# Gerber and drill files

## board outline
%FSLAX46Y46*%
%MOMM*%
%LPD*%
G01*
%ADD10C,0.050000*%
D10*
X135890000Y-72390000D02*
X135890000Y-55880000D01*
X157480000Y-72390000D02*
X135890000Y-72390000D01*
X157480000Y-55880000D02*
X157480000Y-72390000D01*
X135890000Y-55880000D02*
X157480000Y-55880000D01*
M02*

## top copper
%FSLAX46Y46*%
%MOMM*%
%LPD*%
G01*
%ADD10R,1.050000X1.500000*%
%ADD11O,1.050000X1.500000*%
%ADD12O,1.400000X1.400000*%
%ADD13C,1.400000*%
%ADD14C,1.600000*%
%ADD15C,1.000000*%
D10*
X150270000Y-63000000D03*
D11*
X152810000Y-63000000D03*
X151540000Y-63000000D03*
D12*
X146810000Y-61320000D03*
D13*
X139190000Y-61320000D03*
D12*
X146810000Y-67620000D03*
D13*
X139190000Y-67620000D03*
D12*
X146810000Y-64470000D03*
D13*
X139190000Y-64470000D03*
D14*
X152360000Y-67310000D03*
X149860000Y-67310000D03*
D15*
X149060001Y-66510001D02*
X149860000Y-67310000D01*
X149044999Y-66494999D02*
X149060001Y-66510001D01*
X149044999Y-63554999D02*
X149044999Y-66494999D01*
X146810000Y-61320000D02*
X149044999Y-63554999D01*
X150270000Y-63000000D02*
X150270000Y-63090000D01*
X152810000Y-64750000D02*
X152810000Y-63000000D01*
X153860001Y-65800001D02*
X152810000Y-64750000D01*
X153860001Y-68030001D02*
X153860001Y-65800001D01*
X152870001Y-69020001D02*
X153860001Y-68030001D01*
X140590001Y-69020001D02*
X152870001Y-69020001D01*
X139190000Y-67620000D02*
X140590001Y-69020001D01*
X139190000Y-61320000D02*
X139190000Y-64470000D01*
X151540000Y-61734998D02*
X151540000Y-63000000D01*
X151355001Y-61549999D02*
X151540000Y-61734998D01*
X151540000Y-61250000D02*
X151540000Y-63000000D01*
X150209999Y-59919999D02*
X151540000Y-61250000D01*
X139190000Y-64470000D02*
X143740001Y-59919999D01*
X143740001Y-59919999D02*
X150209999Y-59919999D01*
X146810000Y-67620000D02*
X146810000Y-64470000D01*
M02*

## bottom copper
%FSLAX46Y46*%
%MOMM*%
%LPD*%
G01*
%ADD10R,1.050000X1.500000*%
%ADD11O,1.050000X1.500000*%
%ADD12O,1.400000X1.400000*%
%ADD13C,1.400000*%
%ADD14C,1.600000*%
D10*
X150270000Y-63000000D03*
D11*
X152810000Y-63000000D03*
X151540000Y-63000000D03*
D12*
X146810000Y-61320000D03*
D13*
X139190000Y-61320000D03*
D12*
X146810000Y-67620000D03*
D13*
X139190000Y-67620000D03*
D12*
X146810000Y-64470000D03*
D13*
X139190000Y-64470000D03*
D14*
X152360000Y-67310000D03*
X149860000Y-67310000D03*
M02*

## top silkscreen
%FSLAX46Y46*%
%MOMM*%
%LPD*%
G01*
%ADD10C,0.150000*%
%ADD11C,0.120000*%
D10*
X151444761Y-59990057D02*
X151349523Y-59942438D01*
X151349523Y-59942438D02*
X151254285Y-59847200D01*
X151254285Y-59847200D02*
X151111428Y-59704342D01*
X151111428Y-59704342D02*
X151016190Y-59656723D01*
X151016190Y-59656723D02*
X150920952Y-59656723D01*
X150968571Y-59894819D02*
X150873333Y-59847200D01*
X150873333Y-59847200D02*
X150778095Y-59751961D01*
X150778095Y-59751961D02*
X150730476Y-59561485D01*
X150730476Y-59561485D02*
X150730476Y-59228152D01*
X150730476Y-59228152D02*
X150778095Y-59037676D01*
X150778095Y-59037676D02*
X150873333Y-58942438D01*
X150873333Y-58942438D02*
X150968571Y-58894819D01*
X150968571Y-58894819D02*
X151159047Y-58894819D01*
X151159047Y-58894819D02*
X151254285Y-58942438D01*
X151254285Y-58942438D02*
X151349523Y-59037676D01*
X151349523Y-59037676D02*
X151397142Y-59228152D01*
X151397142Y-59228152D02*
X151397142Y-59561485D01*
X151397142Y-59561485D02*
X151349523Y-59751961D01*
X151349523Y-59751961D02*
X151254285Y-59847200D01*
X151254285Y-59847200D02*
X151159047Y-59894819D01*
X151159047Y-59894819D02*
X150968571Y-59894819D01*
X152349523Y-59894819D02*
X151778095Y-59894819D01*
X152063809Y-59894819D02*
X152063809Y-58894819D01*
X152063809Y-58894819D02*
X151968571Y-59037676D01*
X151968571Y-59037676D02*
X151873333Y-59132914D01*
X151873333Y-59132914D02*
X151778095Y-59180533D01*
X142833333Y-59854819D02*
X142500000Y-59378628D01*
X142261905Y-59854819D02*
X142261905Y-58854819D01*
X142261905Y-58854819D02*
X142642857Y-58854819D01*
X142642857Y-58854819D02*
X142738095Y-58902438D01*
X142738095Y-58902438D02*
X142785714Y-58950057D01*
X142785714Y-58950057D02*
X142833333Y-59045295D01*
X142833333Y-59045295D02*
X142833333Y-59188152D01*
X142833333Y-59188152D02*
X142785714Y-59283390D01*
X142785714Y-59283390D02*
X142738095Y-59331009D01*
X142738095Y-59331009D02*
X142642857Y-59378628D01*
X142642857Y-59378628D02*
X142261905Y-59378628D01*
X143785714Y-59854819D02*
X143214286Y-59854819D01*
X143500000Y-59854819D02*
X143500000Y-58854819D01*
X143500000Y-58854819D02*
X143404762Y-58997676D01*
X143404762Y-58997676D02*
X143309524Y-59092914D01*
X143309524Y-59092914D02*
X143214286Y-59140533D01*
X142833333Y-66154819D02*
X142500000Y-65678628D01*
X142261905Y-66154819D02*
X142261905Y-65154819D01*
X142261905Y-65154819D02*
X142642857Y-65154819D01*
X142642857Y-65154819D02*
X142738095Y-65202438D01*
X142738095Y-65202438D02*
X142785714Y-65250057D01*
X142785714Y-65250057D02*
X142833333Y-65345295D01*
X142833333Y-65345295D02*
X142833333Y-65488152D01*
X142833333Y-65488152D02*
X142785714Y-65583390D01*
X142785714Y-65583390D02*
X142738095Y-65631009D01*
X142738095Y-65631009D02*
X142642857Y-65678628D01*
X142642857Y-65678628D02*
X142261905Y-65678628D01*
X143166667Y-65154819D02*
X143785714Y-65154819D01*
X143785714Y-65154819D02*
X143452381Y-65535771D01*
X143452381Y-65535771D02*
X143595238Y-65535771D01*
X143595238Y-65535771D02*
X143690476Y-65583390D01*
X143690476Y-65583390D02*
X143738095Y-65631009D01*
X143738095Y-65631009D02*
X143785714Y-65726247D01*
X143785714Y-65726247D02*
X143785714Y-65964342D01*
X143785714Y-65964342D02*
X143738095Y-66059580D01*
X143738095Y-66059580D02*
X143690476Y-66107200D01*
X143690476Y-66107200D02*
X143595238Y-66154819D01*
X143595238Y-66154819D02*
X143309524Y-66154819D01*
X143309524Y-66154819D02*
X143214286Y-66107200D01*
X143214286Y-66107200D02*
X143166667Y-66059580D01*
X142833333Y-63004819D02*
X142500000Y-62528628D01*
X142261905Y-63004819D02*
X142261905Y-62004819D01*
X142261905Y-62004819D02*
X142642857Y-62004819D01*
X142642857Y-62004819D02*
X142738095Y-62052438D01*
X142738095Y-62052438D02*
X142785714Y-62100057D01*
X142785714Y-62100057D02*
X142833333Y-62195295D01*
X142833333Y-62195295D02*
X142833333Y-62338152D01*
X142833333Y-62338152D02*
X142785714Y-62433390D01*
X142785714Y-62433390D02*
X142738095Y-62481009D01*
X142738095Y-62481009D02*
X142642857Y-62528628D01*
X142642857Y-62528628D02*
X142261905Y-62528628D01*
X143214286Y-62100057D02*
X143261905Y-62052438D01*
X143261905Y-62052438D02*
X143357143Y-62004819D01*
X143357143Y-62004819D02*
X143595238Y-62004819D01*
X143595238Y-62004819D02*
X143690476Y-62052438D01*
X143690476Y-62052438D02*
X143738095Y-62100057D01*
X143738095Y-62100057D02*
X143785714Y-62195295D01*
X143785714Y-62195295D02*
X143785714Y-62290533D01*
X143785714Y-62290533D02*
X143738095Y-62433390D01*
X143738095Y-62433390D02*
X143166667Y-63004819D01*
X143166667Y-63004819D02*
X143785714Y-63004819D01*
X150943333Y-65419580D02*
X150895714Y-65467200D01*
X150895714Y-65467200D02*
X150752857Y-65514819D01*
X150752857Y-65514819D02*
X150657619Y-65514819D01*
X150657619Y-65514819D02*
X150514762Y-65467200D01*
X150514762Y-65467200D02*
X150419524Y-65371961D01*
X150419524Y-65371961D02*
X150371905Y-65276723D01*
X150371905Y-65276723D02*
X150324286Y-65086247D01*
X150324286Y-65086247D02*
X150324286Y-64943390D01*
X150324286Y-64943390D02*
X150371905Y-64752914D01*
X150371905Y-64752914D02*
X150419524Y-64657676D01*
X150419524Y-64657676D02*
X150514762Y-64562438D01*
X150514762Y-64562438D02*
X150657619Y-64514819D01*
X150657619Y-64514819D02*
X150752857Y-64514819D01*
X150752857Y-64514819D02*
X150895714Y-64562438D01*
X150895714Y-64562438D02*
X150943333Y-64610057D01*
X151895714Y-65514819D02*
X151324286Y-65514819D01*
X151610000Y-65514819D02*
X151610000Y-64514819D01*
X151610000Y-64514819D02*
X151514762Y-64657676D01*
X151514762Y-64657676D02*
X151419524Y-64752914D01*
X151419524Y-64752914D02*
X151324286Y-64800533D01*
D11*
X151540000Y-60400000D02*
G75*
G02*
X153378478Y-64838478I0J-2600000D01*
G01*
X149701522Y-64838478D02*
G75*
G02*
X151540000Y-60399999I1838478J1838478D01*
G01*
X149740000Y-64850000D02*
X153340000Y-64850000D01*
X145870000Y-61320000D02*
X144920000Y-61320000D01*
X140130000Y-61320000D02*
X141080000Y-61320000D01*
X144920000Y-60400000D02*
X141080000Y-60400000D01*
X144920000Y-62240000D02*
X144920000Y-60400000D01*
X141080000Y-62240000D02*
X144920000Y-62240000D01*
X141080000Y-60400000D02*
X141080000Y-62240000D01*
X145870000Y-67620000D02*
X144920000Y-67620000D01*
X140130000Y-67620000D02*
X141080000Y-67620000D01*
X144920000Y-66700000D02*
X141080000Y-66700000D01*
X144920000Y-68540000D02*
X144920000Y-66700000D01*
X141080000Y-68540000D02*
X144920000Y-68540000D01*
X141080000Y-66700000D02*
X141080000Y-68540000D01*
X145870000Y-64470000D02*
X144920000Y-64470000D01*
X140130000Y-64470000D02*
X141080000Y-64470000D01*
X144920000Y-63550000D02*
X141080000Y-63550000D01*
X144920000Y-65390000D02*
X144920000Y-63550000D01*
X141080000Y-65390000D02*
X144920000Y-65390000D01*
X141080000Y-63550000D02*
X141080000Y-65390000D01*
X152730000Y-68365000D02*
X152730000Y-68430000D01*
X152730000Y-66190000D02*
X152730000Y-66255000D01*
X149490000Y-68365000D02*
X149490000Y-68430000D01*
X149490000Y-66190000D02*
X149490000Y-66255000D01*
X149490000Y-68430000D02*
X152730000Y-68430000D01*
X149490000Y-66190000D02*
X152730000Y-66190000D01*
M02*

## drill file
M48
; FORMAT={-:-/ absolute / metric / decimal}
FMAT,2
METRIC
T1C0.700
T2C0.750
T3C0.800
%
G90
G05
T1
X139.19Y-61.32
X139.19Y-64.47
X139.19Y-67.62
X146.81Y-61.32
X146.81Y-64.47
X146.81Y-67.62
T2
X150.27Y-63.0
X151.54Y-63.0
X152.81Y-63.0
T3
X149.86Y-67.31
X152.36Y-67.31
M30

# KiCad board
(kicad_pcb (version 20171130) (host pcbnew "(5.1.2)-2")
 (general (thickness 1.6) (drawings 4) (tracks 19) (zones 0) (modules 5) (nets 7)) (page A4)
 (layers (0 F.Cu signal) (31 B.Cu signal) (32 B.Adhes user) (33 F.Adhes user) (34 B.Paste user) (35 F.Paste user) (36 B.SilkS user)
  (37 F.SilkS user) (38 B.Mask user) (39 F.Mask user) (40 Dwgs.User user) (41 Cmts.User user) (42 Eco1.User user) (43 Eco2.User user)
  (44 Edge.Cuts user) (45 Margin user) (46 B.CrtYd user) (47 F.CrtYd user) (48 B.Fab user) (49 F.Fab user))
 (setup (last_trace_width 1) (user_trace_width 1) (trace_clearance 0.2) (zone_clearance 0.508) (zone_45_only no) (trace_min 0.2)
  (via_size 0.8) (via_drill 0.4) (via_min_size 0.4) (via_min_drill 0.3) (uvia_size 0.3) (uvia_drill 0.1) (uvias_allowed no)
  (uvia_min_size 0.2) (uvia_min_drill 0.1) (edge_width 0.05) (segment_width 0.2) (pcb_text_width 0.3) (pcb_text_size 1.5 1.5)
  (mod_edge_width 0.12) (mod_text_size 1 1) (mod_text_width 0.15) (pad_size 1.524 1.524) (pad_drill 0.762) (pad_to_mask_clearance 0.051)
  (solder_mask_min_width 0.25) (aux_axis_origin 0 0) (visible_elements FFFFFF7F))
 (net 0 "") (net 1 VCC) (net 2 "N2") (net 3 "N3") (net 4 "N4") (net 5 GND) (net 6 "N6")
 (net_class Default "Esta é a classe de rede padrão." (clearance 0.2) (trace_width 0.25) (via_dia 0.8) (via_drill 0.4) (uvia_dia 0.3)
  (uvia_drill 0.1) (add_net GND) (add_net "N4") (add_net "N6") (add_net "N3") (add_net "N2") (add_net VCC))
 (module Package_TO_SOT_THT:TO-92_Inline (layer F.Cu) (at 150.27 63)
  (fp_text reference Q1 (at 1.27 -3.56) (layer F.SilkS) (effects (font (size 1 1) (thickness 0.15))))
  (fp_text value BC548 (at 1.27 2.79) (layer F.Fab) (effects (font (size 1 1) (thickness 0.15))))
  (fp_arc (start 1.27 0) (end 1.27 -2.6) (angle 135) (layer F.SilkS) (width 0.12))
  (fp_arc (start 1.27 0) (end 1.27 -2.6) (angle -135) (layer F.SilkS) (width 0.12))
  (fp_line (start -0.53 1.85) (end 3.07 1.85) (layer F.SilkS) (width 0.12))
  (pad 1 thru_hole rect (at 0 0) (size 1.05 1.5) (drill 0.75) (layers *.Cu *.Mask) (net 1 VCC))
  (pad 3 thru_hole oval (at 2.54 0) (size 1.05 1.5) (drill 0.75) (layers *.Cu *.Mask) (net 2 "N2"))
  (pad 2 thru_hole oval (at 1.27 0) (size 1.05 1.5) (drill 0.75) (layers *.Cu *.Mask) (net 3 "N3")))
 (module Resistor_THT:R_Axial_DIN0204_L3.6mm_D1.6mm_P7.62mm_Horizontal (layer F.Cu) (at 139.19 61.32)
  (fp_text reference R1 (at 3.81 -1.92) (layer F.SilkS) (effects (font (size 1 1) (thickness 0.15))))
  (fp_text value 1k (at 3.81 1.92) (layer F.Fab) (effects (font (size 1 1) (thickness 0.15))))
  (fp_line (start 6.68 0) (end 5.73 0) (layer F.SilkS) (width 0.12))
  (fp_line (start 0.94 0) (end 1.89 0) (layer F.SilkS) (width 0.12))
  (fp_line (start 5.73 -0.92) (end 1.89 -0.92) (layer F.SilkS) (width 0.12))
  (fp_line (start 5.73 0.92) (end 5.73 -0.92) (layer F.SilkS) (width 0.12))
  (fp_line (start 1.89 0.92) (end 5.73 0.92) (layer F.SilkS) (width 0.12))
  (fp_line (start 1.89 -0.92) (end 1.89 0.92) (layer F.SilkS) (width 0.12))
  (pad 2 thru_hole oval (at 7.62 0) (size 1.4 1.4) (drill 0.7) (layers *.Cu *.Mask) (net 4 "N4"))
  (pad 1 thru_hole circle (at 0 0) (size 1.4 1.4) (drill 0.7) (layers *.Cu *.Mask) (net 3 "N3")))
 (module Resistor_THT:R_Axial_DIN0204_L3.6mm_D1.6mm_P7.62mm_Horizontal (layer F.Cu) (at 139.19 67.62)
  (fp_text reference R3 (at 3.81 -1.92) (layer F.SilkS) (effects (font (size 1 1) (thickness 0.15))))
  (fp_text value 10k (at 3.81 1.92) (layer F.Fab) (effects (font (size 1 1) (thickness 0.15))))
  (fp_line (start 6.68 0) (end 5.73 0) (layer F.SilkS) (width 0.12))
  (fp_line (start 0.94 0) (end 1.89 0) (layer F.SilkS) (width 0.12))
  (fp_line (start 5.73 -0.92) (end 1.89 -0.92) (layer F.SilkS) (width 0.12))
  (fp_line (start 5.73 0.92) (end 5.73 -0.92) (layer F.SilkS) (width 0.12))
  (fp_line (start 1.89 0.92) (end 5.73 0.92) (layer F.SilkS) (width 0.12))
  (fp_line (start 1.89 -0.92) (end 1.89 0.92) (layer F.SilkS) (width 0.12))
  (pad 2 thru_hole oval (at 7.62 0) (size 1.4 1.4) (drill 0.7) (layers *.Cu *.Mask) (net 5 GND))
  (pad 1 thru_hole circle (at 0 0) (size 1.4 1.4) (drill 0.7) (layers *.Cu *.Mask) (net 2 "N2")))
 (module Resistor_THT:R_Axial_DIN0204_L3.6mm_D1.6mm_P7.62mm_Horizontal (layer F.Cu) (at 139.19 64.47)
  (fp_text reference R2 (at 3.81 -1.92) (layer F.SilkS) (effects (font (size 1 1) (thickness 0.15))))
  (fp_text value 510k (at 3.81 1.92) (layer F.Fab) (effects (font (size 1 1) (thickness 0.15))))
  (fp_line (start 6.68 0) (end 5.73 0) (layer F.SilkS) (width 0.12))
  (fp_line (start 0.94 0) (end 1.89 0) (layer F.SilkS) (width 0.12))
  (fp_line (start 5.73 -0.92) (end 1.89 -0.92) (layer F.SilkS) (width 0.12))
  (fp_line (start 5.73 0.92) (end 5.73 -0.92) (layer F.SilkS) (width 0.12))
  (fp_line (start 1.89 0.92) (end 5.73 0.92) (layer F.SilkS) (width 0.12))
  (fp_line (start 1.89 -0.92) (end 1.89 0.92) (layer F.SilkS) (width 0.12))
  (pad 2 thru_hole oval (at 7.62 0) (size 1.4 1.4) (drill 0.7) (layers *.Cu *.Mask) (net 5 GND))
  (pad 1 thru_hole circle (at 0 0) (size 1.4 1.4) (drill 0.7) (layers *.Cu *.Mask) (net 3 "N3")))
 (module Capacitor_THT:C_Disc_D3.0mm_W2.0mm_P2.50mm (layer F.Cu) (at 149.86 67.31)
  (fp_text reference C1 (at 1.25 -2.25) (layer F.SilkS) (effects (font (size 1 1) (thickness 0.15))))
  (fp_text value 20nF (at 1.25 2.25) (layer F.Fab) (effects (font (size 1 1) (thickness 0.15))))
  (fp_line (start 2.87 1.055) (end 2.87 1.12) (layer F.SilkS) (width 0.12))
  (fp_line (start 2.87 -1.12) (end 2.87 -1.055) (layer F.SilkS) (width 0.12))
  (fp_line (start -0.37 1.055) (end -0.37 1.12) (layer F.SilkS) (width 0.12))
  (fp_line (start -0.37 -1.12) (end -0.37 -1.055) (layer F.SilkS) (width 0.12))
  (fp_line (start -0.37 1.12) (end 2.87 1.12) (layer F.SilkS) (width 0.12))
  (fp_line (start -0.37 -1.12) (end 2.87 -1.12) (layer F.SilkS) (width 0.12))
  (pad 2 thru_hole circle (at 2.5 0) (size 1.6 1.6) (drill 0.8) (layers *.Cu *.Mask) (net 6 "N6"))
  (pad 1 thru_hole circle (at 0 0) (size 1.6 1.6) (drill 0.8) (layers *.Cu *.Mask) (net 4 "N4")))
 (gr_line (start 135.89 72.39) (end 135.89 55.88) (layer Edge.Cuts) (width 0.05))
 (gr_line (start 157.48 72.39) (end 135.89 72.39) (layer Edge.Cuts) (width 0.05))
 (gr_line (start 157.48 55.88) (end 157.48 72.39) (layer Edge.Cuts) (width 0.05))
 (gr_line (start 135.89 55.88) (end 157.48 55.88) (layer Edge.Cuts) (width 0.05))
 (segment (start 149.060001 66.510001) (end 149.86 67.31) (width 1) (layer F.Cu) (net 4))
 (segment (start 149.044999 66.494999) (end 149.060001 66.510001) (width 1) (layer F.Cu) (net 4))
 (segment (start 149.044999 63.554999) (end 149.044999 66.494999) (width 1) (layer F.Cu) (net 4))
 (segment (start 146.81 61.32) (end 149.044999 63.554999) (width 1) (layer F.Cu) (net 4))
 (segment (start 150.27 63) (end 150.27 63.09) (width 1) (layer F.Cu) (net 1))
 (segment (start 152.81 64.75) (end 152.81 63) (width 1) (layer F.Cu) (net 2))
 (segment (start 153.860001 65.800001) (end 152.81 64.75) (width 1) (layer F.Cu) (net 2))
 (segment (start 153.860001 68.030001) (end 153.860001 65.800001) (width 1) (layer F.Cu) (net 2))
 (segment (start 152.870001 69.020001) (end 153.860001 68.030001) (width 1) (layer F.Cu) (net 2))
 (segment (start 140.590001 69.020001) (end 152.870001 69.020001) (width 1) (layer F.Cu) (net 2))
 (segment (start 139.19 67.62) (end 140.590001 69.020001) (width 1) (layer F.Cu) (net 2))
 (segment (start 139.19 61.32) (end 139.19 64.47) (width 1) (layer F.Cu) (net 3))
 (segment (start 151.54 61.734998) (end 151.54 63) (width 1) (layer F.Cu) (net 3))
 (segment (start 151.355001 61.549999) (end 151.54 61.734998) (width 1) (layer F.Cu) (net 3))
 (segment (start 151.54 61.25) (end 151.54 63) (width 1) (layer F.Cu) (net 3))
 (segment (start 150.209999 59.919999) (end 151.54 61.25) (width 1) (layer F.Cu) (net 3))
 (segment (start 139.19 64.47) (end 143.740001 59.919999) (width 1) (layer F.Cu) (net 3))
 (segment (start 143.740001 59.919999) (end 150.209999 59.919999) (width 1) (layer F.Cu) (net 3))
 (segment (start 146.81 67.62) (end 146.81 64.47) (width 1) (layer F.Cu) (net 5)))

